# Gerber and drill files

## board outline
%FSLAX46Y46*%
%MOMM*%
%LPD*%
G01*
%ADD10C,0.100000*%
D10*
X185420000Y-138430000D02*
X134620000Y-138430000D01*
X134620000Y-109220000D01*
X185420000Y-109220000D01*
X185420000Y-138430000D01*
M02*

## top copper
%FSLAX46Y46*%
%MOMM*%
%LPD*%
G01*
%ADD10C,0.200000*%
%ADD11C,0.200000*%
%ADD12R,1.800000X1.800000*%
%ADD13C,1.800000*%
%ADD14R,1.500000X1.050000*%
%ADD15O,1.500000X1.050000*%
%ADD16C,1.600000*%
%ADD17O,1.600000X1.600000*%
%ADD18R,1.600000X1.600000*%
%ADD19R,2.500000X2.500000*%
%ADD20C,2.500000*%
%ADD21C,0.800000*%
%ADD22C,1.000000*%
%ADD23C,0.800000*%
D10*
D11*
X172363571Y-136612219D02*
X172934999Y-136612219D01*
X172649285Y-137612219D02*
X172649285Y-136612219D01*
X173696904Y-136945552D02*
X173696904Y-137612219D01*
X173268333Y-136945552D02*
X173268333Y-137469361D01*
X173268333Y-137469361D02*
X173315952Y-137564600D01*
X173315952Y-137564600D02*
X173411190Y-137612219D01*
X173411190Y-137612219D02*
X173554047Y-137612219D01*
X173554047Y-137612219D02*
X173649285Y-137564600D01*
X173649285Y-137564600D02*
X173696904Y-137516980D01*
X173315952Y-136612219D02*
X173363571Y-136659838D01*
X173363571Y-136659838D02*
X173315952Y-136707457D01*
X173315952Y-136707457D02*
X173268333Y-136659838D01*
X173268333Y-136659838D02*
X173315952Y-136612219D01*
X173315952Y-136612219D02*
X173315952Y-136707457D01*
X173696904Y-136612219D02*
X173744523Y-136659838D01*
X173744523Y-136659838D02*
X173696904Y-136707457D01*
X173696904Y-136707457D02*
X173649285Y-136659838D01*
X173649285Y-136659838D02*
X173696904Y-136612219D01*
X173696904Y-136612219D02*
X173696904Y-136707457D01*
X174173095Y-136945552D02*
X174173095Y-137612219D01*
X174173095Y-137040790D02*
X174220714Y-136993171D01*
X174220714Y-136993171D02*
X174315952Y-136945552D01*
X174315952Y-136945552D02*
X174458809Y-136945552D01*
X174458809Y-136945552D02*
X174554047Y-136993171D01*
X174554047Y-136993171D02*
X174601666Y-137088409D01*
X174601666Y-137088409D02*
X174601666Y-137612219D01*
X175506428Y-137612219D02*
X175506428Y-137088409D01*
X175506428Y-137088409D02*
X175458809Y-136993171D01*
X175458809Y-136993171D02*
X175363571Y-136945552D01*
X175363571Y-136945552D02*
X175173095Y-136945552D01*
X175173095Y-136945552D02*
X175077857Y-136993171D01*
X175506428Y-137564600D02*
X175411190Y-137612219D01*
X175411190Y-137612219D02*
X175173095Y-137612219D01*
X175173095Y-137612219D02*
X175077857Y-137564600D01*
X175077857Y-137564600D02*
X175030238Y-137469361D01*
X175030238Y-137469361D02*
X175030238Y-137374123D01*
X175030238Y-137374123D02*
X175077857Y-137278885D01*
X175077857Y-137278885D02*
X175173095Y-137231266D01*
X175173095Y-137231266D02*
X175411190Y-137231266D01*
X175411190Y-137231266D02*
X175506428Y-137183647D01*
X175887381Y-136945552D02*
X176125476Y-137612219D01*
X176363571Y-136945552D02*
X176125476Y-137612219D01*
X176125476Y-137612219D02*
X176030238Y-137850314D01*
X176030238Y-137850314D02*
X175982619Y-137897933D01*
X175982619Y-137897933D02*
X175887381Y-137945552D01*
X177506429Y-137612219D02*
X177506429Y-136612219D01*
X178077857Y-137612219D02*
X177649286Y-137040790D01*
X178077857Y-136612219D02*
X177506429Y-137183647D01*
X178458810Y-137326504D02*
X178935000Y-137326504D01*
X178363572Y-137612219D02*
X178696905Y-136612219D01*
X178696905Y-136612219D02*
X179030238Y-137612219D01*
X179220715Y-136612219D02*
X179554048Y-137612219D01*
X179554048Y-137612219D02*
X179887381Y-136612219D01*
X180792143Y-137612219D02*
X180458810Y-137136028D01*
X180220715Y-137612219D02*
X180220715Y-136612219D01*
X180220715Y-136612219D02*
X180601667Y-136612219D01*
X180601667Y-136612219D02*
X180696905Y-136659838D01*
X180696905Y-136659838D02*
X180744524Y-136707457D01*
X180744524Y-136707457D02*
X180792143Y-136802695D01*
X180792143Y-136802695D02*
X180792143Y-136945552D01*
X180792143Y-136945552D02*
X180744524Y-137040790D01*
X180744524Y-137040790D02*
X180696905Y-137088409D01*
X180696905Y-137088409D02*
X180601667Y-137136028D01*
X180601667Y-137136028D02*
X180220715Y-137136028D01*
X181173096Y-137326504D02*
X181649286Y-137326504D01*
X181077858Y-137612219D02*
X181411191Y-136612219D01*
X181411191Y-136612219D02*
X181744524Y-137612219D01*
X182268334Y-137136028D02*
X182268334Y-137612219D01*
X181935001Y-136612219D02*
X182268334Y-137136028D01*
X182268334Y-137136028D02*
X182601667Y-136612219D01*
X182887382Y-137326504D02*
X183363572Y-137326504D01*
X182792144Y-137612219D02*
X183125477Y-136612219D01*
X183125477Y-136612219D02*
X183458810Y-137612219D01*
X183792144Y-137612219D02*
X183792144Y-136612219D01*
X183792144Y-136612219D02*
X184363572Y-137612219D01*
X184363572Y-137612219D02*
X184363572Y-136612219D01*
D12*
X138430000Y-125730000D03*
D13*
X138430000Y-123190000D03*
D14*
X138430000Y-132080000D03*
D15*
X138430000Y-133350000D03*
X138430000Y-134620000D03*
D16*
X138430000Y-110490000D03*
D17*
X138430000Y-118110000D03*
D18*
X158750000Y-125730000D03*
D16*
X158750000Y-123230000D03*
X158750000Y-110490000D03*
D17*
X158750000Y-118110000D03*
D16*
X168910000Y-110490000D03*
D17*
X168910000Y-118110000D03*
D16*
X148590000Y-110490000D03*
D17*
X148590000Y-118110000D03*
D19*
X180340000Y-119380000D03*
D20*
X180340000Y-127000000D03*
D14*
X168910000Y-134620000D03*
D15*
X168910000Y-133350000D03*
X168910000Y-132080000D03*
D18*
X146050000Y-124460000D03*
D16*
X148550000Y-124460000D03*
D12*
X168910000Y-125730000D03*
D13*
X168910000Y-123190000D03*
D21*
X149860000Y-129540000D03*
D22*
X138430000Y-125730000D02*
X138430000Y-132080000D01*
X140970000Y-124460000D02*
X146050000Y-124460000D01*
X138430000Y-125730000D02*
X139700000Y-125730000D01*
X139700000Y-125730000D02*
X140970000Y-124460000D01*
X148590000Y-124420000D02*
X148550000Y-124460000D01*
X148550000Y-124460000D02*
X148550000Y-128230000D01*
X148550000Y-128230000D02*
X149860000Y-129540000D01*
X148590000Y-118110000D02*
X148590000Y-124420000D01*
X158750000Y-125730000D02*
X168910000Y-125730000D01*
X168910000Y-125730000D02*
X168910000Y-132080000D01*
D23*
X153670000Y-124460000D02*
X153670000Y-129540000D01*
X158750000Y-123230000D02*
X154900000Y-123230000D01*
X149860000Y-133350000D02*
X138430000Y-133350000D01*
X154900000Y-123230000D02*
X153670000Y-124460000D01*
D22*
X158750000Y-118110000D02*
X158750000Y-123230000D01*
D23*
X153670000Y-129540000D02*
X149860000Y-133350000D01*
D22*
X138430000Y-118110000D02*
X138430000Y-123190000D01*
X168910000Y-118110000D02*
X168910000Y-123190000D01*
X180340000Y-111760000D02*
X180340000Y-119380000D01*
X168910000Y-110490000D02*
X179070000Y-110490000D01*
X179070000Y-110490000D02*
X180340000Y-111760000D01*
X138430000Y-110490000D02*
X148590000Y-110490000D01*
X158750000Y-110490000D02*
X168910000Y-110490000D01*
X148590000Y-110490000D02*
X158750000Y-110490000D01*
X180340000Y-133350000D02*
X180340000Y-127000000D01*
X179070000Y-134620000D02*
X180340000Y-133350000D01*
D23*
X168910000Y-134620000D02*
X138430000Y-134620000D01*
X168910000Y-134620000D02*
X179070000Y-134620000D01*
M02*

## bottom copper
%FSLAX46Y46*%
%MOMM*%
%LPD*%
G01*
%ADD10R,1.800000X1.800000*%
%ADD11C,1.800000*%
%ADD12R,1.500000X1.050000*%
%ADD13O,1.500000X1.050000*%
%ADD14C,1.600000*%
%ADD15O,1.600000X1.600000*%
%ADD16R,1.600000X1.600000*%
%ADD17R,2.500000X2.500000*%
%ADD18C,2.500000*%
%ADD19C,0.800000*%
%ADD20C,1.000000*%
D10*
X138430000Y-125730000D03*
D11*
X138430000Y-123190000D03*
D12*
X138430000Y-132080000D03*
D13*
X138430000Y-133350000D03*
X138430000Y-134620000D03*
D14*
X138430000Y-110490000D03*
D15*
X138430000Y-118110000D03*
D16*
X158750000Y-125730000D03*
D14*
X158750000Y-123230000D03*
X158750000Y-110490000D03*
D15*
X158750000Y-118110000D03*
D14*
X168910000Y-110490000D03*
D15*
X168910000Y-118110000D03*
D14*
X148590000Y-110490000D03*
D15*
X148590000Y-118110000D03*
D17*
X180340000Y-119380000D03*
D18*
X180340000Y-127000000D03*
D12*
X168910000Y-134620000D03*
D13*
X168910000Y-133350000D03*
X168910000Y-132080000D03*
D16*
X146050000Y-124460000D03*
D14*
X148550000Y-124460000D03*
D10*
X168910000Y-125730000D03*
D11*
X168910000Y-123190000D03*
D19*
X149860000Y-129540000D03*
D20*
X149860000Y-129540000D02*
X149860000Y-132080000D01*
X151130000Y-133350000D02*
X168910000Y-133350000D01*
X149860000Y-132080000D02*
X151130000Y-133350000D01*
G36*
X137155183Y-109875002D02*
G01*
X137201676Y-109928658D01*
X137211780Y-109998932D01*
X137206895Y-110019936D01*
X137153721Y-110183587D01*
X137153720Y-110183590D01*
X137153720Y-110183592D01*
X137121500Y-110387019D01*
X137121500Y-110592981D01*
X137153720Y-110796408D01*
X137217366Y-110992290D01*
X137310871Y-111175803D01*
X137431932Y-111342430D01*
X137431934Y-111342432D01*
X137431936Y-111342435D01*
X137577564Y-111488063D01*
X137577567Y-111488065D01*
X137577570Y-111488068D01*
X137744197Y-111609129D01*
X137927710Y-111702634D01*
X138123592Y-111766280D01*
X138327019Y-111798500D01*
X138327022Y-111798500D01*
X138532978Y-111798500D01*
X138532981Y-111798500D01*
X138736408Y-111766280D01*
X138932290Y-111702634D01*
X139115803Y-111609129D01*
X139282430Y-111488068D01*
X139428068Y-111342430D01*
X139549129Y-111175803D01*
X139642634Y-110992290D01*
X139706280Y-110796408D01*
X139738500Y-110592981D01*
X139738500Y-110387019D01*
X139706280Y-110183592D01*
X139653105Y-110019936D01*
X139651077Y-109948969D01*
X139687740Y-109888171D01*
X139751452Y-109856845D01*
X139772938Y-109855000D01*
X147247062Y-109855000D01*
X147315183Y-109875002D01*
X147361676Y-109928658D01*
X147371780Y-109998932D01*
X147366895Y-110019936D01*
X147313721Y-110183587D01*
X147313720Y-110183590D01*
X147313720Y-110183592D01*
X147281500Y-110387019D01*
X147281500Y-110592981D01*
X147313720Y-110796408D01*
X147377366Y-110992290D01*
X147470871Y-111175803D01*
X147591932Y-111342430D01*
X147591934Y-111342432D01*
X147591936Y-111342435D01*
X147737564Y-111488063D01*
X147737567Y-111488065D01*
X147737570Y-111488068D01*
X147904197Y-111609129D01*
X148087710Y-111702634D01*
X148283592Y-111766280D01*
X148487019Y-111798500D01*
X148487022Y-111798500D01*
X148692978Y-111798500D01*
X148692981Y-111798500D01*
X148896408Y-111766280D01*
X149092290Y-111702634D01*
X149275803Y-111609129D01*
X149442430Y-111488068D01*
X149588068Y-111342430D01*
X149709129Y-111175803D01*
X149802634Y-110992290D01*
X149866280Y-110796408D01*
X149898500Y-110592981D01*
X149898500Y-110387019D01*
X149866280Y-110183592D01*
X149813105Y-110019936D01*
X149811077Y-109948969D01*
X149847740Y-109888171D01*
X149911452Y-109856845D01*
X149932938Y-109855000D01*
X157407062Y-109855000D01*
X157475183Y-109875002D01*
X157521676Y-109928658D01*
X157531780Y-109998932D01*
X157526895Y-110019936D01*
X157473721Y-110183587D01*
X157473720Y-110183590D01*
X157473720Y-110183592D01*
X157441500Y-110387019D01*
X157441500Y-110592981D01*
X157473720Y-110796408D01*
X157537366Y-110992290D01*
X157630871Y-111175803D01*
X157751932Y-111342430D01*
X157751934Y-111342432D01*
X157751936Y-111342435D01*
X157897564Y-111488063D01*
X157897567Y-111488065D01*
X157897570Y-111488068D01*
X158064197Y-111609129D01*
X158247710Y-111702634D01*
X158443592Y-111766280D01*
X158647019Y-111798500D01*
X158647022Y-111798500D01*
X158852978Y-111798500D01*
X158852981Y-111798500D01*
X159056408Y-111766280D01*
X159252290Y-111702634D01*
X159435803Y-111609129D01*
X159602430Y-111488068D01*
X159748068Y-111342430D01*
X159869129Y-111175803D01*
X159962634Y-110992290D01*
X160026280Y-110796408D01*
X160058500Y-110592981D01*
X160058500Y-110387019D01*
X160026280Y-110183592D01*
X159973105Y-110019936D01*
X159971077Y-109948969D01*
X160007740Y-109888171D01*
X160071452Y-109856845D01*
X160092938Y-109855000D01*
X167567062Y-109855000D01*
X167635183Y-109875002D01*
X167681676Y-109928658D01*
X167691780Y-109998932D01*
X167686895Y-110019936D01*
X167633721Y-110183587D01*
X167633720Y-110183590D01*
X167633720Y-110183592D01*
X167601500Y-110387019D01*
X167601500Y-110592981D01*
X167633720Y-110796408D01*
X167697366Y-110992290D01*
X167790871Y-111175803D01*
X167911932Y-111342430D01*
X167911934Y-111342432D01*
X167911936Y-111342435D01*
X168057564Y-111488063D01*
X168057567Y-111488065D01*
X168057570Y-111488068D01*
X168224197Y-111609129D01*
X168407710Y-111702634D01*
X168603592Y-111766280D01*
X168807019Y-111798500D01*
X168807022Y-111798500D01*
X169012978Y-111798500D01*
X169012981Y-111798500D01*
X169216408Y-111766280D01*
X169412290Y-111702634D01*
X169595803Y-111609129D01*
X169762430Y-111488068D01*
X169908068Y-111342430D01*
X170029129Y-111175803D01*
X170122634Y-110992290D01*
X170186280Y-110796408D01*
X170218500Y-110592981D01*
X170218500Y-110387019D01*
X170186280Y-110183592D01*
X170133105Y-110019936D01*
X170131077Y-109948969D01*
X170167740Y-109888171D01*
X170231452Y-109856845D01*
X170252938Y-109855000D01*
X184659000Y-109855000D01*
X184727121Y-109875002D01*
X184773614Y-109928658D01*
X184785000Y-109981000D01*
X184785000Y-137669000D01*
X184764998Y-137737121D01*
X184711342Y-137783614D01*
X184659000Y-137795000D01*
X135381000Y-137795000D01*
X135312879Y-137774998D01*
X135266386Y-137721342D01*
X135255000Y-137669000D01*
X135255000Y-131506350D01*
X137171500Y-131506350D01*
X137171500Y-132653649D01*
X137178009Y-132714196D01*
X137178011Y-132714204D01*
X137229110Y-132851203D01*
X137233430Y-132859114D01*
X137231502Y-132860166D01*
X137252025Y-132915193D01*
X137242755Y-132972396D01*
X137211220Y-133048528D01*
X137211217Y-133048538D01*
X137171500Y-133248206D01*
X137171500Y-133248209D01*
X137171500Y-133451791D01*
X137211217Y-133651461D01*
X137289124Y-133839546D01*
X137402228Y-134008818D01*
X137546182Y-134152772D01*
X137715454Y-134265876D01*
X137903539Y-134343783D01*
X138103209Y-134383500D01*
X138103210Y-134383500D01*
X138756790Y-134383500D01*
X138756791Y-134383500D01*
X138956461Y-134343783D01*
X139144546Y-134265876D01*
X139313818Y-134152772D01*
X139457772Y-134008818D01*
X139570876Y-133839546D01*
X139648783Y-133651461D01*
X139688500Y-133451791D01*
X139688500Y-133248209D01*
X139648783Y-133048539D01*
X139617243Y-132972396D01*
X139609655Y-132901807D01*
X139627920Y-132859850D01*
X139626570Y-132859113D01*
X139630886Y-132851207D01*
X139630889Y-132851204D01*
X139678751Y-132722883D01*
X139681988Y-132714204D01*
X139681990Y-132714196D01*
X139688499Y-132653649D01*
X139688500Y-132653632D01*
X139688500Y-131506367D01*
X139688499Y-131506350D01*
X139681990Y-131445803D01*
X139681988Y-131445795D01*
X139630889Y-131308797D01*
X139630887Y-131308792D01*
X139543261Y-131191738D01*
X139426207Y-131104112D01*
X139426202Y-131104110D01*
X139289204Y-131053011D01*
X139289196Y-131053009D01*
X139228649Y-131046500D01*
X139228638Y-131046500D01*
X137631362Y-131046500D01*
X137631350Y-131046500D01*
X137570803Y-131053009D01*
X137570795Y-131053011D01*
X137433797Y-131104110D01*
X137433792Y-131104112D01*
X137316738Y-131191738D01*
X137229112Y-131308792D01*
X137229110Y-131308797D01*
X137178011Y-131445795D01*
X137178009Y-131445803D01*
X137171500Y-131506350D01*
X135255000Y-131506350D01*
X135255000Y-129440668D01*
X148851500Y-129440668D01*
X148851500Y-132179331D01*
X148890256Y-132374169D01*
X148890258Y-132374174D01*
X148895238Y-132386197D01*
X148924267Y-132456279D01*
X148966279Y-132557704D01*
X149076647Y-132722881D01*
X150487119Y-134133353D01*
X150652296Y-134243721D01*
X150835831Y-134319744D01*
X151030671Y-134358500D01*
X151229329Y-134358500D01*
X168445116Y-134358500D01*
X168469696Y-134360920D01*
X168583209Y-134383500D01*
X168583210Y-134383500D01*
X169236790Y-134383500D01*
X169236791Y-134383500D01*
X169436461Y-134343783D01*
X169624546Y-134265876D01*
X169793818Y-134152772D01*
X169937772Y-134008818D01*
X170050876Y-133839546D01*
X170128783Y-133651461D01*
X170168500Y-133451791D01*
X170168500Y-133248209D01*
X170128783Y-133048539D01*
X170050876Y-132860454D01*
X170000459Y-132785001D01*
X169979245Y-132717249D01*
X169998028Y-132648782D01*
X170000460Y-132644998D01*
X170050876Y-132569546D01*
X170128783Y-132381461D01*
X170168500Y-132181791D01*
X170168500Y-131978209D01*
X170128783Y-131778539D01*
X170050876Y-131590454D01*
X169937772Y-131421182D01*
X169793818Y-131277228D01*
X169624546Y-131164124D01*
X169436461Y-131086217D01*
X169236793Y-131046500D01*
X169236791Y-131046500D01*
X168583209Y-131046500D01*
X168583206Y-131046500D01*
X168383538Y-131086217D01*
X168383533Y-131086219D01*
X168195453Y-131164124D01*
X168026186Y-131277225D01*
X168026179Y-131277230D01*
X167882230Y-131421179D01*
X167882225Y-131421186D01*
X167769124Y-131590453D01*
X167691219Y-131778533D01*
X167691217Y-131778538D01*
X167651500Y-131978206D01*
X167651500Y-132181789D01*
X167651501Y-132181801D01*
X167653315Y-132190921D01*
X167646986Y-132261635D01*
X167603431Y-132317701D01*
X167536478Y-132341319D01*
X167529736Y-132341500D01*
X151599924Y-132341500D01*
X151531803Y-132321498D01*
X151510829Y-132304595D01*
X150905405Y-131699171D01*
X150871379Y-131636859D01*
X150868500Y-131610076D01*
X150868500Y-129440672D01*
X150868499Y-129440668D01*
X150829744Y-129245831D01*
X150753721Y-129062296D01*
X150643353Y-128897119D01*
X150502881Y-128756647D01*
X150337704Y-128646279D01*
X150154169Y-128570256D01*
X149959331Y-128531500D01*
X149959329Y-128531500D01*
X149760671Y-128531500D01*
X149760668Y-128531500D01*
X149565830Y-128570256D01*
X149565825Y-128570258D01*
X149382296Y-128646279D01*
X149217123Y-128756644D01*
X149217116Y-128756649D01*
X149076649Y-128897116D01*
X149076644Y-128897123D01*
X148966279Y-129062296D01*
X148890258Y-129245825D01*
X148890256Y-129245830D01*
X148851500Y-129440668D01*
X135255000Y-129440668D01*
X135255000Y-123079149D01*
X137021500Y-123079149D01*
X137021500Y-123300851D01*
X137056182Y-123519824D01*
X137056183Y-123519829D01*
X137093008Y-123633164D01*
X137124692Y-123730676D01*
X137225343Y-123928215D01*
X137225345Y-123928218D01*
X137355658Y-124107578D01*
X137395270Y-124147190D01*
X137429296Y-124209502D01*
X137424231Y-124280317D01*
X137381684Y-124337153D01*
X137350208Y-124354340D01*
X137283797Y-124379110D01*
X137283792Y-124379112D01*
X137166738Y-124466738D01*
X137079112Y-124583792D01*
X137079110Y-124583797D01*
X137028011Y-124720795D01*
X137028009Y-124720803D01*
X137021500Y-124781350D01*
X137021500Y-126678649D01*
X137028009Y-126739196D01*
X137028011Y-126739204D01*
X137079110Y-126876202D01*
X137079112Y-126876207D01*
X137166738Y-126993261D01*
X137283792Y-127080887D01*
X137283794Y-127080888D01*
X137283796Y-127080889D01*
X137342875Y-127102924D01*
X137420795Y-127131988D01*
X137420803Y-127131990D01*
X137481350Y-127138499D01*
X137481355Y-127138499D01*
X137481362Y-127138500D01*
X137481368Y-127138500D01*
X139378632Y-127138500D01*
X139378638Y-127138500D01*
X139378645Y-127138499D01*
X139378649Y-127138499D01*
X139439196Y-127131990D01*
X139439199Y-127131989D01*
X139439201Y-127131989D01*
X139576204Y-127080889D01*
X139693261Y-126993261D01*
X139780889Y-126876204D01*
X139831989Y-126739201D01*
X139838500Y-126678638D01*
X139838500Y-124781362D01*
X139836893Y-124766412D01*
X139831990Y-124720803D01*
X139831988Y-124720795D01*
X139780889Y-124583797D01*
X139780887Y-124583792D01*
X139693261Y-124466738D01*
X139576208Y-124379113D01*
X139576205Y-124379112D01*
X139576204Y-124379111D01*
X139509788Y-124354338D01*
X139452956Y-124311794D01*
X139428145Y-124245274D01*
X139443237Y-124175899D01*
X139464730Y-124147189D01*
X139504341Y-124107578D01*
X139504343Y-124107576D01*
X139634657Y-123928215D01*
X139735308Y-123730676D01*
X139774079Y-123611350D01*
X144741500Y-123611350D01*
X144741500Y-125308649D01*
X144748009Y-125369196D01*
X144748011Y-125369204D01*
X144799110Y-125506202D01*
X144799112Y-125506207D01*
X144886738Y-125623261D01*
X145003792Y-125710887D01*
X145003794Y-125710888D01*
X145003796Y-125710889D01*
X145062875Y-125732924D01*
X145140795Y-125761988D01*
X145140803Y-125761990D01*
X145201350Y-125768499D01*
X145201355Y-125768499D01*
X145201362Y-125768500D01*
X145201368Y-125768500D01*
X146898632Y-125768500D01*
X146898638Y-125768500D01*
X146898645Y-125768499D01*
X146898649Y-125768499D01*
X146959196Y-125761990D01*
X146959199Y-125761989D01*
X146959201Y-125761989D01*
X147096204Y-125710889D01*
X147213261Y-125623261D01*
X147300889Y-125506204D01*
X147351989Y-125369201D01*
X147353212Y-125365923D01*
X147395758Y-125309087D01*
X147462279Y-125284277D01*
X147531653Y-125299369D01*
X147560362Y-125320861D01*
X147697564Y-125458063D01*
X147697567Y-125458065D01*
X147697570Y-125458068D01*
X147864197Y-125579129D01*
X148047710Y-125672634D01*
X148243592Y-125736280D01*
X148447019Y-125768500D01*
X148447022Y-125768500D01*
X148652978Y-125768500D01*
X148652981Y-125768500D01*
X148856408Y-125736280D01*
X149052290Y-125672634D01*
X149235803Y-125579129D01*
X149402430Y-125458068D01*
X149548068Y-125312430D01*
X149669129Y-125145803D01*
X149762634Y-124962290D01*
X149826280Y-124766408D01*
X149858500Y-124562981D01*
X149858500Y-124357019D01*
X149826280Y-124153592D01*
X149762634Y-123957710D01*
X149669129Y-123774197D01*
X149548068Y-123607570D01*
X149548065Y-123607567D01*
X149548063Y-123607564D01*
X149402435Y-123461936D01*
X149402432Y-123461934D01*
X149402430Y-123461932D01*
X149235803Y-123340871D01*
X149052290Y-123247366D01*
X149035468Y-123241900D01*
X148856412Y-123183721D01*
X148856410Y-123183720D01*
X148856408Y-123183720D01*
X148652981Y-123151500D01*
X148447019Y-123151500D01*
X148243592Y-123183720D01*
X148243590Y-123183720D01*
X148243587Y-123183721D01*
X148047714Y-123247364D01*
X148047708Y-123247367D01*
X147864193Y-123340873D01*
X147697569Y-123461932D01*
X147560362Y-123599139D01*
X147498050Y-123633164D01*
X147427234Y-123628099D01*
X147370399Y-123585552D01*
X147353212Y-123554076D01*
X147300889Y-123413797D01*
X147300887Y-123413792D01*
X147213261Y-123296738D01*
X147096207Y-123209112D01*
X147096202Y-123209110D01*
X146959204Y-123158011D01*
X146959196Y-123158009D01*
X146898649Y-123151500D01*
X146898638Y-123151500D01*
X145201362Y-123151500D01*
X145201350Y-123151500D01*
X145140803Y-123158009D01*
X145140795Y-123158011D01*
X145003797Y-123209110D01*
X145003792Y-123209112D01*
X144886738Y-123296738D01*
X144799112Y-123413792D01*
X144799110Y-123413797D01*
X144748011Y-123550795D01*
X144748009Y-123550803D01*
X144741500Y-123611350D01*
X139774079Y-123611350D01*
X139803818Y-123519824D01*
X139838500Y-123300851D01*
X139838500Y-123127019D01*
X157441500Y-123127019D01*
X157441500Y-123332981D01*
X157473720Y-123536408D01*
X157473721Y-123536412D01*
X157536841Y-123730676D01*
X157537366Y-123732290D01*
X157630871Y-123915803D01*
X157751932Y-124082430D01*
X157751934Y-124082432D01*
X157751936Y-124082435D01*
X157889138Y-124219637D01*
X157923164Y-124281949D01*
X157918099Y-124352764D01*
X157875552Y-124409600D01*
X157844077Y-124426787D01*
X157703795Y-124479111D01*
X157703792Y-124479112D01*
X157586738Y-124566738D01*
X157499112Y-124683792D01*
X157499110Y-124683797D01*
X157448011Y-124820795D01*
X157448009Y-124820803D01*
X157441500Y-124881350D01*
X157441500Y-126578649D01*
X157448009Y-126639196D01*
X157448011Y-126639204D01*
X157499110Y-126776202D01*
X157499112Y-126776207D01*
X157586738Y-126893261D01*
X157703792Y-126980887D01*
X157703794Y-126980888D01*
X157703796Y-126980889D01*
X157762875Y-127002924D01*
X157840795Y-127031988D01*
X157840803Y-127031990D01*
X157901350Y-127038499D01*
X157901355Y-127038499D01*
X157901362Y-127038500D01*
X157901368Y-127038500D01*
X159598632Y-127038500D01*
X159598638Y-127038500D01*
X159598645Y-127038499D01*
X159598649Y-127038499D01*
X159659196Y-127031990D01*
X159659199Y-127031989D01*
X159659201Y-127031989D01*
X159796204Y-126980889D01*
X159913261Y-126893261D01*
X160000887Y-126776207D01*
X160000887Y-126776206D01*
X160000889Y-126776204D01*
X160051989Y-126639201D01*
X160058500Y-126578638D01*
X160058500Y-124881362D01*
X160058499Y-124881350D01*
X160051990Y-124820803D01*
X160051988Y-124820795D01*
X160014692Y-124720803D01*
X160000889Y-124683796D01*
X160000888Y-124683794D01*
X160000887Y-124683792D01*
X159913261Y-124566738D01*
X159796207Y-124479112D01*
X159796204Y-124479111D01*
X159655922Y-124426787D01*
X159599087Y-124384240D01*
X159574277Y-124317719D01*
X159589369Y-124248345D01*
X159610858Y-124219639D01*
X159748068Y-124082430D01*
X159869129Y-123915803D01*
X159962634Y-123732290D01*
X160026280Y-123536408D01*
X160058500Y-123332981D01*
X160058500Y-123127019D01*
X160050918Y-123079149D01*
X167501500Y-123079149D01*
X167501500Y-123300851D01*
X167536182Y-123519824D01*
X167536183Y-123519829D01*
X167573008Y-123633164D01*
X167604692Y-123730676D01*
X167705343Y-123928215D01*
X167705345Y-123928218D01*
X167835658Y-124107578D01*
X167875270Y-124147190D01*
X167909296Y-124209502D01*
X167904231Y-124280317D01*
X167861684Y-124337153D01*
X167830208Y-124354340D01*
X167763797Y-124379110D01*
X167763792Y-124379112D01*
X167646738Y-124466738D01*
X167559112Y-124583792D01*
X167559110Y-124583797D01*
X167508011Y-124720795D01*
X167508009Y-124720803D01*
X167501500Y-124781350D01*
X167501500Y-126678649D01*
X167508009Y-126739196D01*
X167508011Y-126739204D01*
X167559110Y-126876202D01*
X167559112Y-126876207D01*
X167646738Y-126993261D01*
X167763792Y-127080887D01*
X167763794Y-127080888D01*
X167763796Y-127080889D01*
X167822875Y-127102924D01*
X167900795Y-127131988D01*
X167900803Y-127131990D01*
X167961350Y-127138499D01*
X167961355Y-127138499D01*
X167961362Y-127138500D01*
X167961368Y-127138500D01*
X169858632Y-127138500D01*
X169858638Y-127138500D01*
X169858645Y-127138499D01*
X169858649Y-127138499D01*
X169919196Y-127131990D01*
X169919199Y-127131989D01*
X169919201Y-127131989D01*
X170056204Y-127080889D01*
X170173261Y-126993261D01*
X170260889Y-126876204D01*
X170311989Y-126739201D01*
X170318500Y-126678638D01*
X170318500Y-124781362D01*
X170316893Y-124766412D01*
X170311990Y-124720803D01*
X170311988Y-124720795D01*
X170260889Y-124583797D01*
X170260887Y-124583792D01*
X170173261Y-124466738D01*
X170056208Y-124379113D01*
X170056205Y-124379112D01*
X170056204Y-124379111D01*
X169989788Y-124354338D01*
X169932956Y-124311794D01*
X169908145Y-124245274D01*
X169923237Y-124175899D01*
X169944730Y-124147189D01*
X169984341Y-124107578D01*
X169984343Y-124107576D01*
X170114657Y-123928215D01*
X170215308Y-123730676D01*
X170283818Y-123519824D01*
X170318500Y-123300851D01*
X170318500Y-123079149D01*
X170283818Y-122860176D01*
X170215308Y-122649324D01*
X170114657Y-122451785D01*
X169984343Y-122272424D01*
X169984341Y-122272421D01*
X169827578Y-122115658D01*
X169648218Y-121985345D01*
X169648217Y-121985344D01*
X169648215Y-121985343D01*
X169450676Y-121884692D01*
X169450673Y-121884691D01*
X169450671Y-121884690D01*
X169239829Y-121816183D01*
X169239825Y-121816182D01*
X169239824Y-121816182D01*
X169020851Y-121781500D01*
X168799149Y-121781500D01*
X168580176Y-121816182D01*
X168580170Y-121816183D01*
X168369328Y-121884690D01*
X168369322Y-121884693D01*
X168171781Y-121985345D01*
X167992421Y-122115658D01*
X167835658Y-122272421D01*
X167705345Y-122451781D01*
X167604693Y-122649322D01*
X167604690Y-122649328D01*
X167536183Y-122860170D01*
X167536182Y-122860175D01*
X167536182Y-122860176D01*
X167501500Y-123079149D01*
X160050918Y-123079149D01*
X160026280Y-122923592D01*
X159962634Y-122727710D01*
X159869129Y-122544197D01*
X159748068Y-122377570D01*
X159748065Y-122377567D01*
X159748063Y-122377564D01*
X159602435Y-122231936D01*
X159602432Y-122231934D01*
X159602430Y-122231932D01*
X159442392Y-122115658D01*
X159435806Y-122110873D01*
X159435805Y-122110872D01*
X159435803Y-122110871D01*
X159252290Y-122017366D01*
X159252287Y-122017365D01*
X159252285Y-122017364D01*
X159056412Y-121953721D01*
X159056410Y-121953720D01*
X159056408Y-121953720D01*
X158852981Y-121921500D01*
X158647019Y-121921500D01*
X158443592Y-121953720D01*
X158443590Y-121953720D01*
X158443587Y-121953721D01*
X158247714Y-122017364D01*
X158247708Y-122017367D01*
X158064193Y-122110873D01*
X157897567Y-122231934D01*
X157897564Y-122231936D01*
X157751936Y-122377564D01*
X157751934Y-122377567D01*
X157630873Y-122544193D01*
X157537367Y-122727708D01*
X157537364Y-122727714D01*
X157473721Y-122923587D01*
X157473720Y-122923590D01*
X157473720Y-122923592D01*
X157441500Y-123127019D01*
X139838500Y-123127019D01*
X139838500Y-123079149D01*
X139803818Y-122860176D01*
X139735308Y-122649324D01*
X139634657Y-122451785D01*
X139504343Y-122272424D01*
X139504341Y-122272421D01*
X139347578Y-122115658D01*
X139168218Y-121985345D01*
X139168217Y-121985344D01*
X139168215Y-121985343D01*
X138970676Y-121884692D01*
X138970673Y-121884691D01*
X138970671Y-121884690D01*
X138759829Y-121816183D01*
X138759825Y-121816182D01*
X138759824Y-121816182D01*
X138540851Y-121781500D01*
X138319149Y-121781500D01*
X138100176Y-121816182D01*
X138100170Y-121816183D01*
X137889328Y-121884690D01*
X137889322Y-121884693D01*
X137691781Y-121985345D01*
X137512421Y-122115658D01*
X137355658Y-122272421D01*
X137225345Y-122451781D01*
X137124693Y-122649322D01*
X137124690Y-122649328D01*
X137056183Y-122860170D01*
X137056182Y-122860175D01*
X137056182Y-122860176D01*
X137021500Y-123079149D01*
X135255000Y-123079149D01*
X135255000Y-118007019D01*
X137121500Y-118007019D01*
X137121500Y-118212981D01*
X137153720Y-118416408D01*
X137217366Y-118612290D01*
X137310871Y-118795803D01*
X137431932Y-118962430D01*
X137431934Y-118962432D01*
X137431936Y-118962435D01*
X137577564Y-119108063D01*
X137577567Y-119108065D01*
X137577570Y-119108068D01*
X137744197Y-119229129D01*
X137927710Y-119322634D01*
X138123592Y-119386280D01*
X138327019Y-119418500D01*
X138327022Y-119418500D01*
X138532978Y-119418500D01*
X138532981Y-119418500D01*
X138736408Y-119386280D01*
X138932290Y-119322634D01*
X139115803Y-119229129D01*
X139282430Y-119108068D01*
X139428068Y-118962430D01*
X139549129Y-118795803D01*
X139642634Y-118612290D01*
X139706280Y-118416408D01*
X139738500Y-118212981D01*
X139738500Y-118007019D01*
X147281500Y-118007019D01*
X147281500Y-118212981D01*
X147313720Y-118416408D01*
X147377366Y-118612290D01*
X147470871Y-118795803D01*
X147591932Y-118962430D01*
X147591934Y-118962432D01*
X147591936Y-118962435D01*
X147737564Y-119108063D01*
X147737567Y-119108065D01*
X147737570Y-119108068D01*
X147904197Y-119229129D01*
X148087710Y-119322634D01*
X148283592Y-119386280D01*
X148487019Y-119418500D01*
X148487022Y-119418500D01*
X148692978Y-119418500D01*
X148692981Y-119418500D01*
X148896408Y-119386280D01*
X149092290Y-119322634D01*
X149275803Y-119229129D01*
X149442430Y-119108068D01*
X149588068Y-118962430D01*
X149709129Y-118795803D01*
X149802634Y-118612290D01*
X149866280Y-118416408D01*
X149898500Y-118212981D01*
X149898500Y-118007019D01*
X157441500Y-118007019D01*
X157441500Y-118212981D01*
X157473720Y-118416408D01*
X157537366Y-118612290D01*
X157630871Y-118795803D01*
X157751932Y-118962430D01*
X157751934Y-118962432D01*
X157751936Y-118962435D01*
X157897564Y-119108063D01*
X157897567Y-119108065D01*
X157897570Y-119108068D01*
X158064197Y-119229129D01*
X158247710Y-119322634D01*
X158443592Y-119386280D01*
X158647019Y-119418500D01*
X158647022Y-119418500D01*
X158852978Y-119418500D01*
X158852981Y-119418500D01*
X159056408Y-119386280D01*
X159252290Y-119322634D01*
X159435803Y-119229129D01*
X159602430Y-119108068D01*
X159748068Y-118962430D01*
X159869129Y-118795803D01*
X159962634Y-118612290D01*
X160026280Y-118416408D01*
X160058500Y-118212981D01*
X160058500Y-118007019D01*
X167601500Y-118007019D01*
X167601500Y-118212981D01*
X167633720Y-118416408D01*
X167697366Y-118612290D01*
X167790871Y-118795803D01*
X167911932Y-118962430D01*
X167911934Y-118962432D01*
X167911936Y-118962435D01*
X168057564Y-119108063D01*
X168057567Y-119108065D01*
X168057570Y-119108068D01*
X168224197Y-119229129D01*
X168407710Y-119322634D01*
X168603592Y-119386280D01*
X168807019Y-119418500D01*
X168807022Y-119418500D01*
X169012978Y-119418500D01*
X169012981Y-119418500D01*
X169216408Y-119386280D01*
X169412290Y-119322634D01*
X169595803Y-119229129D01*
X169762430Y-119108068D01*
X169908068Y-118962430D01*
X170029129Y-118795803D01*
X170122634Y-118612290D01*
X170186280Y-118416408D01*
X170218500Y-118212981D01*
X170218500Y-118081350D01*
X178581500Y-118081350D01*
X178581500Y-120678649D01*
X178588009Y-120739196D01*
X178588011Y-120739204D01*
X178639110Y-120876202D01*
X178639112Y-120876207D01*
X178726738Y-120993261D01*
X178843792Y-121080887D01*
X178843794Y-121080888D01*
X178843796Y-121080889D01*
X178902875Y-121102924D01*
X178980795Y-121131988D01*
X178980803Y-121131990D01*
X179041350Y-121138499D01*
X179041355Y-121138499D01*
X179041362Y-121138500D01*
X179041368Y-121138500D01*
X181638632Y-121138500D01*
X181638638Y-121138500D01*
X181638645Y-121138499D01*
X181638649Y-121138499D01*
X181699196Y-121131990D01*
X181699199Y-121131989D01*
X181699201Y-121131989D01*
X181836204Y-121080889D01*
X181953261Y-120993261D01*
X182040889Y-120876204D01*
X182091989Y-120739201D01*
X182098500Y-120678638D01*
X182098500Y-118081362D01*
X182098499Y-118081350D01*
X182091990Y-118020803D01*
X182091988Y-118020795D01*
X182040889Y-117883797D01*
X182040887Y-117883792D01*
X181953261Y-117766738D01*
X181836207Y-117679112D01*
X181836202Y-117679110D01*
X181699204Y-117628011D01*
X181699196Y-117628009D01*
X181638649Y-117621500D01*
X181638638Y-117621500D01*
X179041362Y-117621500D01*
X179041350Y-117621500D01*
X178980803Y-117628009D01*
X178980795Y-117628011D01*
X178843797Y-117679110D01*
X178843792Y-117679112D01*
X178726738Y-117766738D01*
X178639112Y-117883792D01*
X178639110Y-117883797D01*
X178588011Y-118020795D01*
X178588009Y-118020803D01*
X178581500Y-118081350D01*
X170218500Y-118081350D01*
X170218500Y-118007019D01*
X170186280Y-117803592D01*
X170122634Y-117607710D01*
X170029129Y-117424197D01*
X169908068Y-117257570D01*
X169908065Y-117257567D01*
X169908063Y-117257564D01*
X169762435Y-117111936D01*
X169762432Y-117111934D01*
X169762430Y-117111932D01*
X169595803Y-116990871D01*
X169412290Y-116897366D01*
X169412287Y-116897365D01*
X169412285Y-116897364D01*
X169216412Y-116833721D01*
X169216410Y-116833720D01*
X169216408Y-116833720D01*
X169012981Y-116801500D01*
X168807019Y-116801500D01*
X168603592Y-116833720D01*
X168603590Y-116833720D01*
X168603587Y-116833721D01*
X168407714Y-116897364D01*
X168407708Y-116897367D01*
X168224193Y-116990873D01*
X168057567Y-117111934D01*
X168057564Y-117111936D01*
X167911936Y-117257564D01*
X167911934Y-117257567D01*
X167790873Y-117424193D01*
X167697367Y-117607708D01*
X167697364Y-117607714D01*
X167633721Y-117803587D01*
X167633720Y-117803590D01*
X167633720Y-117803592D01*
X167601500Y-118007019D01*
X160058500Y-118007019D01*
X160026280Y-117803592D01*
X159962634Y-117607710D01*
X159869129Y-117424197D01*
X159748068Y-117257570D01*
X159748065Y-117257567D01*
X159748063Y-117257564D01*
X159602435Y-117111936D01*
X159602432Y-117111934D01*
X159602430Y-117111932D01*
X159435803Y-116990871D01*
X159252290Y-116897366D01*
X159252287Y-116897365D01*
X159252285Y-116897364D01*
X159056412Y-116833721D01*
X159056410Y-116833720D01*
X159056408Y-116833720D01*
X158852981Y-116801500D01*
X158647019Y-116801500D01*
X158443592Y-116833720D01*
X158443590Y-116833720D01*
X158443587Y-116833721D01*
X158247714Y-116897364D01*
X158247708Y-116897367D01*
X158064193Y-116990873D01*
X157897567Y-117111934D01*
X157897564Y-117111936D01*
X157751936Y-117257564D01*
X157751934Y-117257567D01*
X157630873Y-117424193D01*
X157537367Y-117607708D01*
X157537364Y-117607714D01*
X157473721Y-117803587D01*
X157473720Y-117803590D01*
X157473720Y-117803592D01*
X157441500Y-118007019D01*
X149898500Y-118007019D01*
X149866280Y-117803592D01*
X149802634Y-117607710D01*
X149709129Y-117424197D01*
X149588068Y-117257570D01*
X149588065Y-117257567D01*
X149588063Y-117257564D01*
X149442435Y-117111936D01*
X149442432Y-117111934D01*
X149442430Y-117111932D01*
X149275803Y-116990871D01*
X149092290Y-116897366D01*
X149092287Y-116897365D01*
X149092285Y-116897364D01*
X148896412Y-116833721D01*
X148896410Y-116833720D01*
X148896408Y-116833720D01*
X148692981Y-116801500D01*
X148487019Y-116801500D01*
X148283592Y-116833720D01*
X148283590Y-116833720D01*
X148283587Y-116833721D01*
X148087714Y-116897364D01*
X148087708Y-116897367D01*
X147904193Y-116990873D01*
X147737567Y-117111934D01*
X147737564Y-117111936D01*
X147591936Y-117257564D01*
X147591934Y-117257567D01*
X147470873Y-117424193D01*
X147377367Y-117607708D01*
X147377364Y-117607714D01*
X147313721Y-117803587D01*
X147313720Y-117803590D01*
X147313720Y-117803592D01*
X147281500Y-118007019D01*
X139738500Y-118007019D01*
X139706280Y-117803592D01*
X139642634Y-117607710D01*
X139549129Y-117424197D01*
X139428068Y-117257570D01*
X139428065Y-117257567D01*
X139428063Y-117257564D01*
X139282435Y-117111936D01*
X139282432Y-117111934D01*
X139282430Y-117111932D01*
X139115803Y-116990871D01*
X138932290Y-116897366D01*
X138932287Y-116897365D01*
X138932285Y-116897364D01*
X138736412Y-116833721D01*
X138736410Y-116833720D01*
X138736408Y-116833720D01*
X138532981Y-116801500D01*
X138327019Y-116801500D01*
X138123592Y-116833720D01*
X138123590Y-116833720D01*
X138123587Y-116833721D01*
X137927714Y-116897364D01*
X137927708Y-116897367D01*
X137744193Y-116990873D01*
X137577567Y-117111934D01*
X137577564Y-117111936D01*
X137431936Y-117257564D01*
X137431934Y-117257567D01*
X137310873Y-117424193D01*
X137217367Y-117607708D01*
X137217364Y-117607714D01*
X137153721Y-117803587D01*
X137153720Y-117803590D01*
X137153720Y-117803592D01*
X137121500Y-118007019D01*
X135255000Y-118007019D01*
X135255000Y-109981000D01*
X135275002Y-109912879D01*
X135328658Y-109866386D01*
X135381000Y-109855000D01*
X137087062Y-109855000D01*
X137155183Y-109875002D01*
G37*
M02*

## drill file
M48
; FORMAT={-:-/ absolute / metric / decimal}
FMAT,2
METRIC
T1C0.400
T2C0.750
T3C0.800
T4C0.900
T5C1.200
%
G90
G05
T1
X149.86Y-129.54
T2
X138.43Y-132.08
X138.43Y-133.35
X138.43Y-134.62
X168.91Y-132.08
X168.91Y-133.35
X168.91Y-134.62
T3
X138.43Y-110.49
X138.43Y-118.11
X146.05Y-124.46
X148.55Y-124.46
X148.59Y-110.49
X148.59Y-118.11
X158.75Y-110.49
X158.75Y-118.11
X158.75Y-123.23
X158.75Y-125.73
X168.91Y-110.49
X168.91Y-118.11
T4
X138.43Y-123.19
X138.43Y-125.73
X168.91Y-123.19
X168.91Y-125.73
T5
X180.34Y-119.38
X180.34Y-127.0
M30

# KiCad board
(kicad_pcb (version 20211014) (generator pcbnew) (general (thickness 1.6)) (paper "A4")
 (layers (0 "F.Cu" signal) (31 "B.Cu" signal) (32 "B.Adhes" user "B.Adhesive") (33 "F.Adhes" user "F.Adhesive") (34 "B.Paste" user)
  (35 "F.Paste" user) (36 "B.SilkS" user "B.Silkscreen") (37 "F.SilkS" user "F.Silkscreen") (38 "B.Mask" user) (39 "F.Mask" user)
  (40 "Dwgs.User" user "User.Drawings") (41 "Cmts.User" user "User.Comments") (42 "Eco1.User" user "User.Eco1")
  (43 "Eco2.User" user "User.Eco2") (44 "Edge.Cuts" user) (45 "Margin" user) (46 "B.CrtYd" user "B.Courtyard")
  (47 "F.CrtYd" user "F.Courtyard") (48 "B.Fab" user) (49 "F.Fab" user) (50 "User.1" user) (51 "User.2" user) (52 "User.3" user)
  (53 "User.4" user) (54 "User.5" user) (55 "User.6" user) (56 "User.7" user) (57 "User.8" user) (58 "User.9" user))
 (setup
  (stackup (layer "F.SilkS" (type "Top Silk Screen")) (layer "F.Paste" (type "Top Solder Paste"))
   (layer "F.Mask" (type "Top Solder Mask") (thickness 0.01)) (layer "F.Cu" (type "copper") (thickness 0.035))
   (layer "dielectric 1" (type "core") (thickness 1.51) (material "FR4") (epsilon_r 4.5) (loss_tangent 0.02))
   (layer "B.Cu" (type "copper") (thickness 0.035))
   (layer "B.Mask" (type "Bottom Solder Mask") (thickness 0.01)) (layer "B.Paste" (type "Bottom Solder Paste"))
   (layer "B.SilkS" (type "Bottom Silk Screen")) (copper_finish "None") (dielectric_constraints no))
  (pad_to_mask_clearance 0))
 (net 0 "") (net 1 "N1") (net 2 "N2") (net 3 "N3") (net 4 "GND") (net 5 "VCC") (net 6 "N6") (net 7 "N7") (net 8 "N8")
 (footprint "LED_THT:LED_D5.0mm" (layer "F.Cu") (at 138.43 125.73 90)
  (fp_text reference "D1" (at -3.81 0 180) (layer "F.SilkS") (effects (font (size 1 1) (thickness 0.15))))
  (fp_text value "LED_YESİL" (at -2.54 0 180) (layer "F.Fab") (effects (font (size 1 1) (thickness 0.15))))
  (pad "1" thru_hole rect (at 0 0 90) (size 1.8 1.8) (drill 0.9) (layers *.Cu *.Mask) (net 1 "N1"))
  (pad "2" thru_hole circle (at 2.54 0 90) (size 1.8 1.8) (drill 0.9) (layers *.Cu *.Mask) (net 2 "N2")))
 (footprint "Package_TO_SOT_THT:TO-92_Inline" (layer "F.Cu") (at 138.43 132.08 -90)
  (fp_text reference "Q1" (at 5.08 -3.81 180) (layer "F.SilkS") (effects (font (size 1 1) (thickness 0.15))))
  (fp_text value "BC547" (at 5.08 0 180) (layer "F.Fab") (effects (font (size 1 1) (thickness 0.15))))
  (pad "1" thru_hole rect (at 0 0 270) (size 1.05 1.5) (drill 0.75) (layers *.Cu *.Mask) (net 1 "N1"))
  (pad "2" thru_hole oval (at 1.27 0 270) (size 1.05 1.5) (drill 0.75) (layers *.Cu *.Mask) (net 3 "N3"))
  (pad "3" thru_hole oval (at 2.54 0 270) (size 1.05 1.5) (drill 0.75) (layers *.Cu *.Mask) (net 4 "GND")))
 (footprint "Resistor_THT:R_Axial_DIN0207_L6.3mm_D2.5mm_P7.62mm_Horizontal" (layer "F.Cu") (at 138.43 110.49 -90)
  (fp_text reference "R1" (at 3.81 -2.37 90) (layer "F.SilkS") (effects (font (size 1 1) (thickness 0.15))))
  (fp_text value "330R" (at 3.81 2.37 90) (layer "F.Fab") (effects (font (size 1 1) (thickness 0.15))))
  (pad "1" thru_hole circle (at 0 0 270) (size 1.6 1.6) (drill 0.8) (layers *.Cu *.Mask) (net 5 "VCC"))
  (pad "2" thru_hole oval (at 7.62 0 270) (size 1.6 1.6) (drill 0.8) (layers *.Cu *.Mask) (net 2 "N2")))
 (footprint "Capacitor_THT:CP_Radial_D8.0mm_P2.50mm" (layer "F.Cu") (at 158.75 125.73 90)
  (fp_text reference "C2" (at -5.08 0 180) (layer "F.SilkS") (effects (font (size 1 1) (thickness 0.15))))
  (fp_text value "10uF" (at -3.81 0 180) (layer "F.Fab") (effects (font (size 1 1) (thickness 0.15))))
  (pad "1" thru_hole rect (at 0 0 90) (size 1.6 1.6) (drill 0.8) (layers *.Cu *.Mask) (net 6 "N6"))
  (pad "2" thru_hole circle (at 2.5 0 90) (size 1.6 1.6) (drill 0.8) (layers *.Cu *.Mask) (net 3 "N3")))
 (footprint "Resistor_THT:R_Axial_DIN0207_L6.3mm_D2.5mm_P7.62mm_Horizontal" (layer "F.Cu") (at 158.75 110.49 -90)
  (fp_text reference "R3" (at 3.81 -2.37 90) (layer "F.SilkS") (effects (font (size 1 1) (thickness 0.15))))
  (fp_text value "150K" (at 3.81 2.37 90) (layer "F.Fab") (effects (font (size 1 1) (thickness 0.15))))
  (pad "1" thru_hole circle (at 0 0 270) (size 1.6 1.6) (drill 0.8) (layers *.Cu *.Mask) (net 5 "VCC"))
  (pad "2" thru_hole oval (at 7.62 0 270) (size 1.6 1.6) (drill 0.8) (layers *.Cu *.Mask) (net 3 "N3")))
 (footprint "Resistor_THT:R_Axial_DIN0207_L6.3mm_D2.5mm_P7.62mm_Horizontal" (layer "F.Cu") (at 168.91 110.49 -90)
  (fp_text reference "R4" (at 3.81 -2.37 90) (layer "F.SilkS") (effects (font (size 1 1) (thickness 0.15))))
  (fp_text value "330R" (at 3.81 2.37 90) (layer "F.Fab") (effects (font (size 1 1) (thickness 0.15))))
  (pad "1" thru_hole circle (at 0 0 270) (size 1.6 1.6) (drill 0.8) (layers *.Cu *.Mask) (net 5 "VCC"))
  (pad "2" thru_hole oval (at 7.62 0 270) (size 1.6 1.6) (drill 0.8) (layers *.Cu *.Mask) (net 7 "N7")))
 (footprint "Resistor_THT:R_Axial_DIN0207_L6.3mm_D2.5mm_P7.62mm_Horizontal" (layer "F.Cu") (at 148.59 110.49 -90)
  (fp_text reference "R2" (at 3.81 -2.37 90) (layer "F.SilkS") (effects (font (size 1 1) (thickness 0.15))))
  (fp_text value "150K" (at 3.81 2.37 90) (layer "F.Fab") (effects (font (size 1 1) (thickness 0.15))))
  (pad "1" thru_hole circle (at 0 0 270) (size 1.6 1.6) (drill 0.8) (layers *.Cu *.Mask) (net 5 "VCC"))
  (pad "2" thru_hole oval (at 7.62 0 270) (size 1.6 1.6) (drill 0.8) (layers *.Cu *.Mask) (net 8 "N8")))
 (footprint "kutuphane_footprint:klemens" (layer "F.Cu") (at 180.34 121.92 -90)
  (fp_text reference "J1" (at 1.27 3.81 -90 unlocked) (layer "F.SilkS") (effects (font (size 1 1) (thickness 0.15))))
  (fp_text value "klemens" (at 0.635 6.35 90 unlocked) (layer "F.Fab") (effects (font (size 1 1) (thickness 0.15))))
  (pad "1" thru_hole rect (at -2.54 0 270) (size 2.5 2.5) (drill 1.2) (layers *.Cu *.Mask) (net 5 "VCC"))
  (pad "2" thru_hole circle (at 5.08 0 270) (size 2.5 2.5) (drill 1.2) (layers *.Cu *.Mask) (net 4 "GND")))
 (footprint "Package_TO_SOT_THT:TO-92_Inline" (layer "F.Cu") (at 168.91 134.62 90)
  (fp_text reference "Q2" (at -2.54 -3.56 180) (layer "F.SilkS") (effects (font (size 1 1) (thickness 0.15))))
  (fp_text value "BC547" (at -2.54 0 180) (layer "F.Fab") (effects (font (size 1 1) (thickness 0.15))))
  (pad "1" thru_hole rect (at 0 0 90) (size 1.05 1.5) (drill 0.75) (layers *.Cu *.Mask) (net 4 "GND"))
  (pad "2" thru_hole oval (at 1.27 0 90) (size 1.05 1.5) (drill 0.75) (layers *.Cu *.Mask) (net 8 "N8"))
  (pad "3" thru_hole oval (at 2.54 0 90) (size 1.05 1.5) (drill 0.75) (layers *.Cu *.Mask) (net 6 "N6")))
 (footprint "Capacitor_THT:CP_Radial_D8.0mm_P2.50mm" (layer "F.Cu") (at 146.05 124.46)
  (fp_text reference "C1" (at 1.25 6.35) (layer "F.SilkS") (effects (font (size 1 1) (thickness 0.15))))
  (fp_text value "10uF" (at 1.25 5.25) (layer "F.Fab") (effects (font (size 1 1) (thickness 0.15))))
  (pad "1" thru_hole rect (at 0 0) (size 1.6 1.6) (drill 0.8) (layers *.Cu *.Mask) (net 1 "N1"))
  (pad "2" thru_hole circle (at 2.5 0) (size 1.6 1.6) (drill 0.8) (layers *.Cu *.Mask) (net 8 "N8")))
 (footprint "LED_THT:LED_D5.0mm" (layer "F.Cu") (at 168.91 125.73 90)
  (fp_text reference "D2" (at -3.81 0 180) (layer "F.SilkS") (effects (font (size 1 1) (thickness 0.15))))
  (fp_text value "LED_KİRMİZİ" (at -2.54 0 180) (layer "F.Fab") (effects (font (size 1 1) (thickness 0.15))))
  (pad "1" thru_hole rect (at 0 0 90) (size 1.8 1.8) (drill 0.9) (layers *.Cu *.Mask) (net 6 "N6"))
  (pad "2" thru_hole circle (at 2.54 0 90) (size 1.8 1.8) (drill 0.9) (layers *.Cu *.Mask) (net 7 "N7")))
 (gr_poly (pts (xy 185.42 138.43) (xy 134.62 138.43) (xy 134.62 109.22) (xy 185.42 109.22)) (layer "Edge.Cuts") (width 0.1) (fill none))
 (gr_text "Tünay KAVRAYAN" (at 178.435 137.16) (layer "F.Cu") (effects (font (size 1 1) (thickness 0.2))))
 (segment (start 138.43 125.73) (end 138.43 132.08) (width 1) (layer "F.Cu") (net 1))
 (segment (start 140.97 124.46) (end 146.05 124.46) (width 1) (layer "F.Cu") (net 1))
 (segment (start 138.43 125.73) (end 139.7 125.73) (width 1) (layer "F.Cu") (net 1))
 (segment (start 139.7 125.73) (end 140.97 124.46) (width 1) (layer "F.Cu") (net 1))
 (segment (start 148.59 124.42) (end 148.55 124.46) (width 1) (layer "F.Cu") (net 8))
 (segment (start 148.55 124.46) (end 148.55 128.23) (width 1) (layer "F.Cu") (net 8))
 (segment (start 148.55 128.23) (end 149.86 129.54) (width 1) (layer "F.Cu") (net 8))
 (segment (start 148.59 118.11) (end 148.59 124.42) (width 1) (layer "F.Cu") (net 8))
 (via (at 149.86 129.54) (size 0.8) (drill 0.4) (layers "F.Cu" "B.Cu") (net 8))
 (segment (start 149.86 129.54) (end 149.86 132.08) (width 1) (layer "B.Cu") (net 8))
 (segment (start 151.13 133.35) (end 168.91 133.35) (width 1) (layer "B.Cu") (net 8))
 (segment (start 149.86 132.08) (end 151.13 133.35) (width 1) (layer "B.Cu") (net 8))
 (segment (start 158.75 125.73) (end 168.91 125.73) (width 1) (layer "F.Cu") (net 6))
 (segment (start 168.91 125.73) (end 168.91 132.08) (width 1) (layer "F.Cu") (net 6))
 (segment (start 153.67 124.46) (end 153.67 129.54) (width 0.8) (layer "F.Cu") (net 3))
 (segment (start 158.75 123.23) (end 154.9 123.23) (width 0.8) (layer "F.Cu") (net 3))
 (segment (start 149.86 133.35) (end 138.43 133.35) (width 0.8) (layer "F.Cu") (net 3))
 (segment (start 154.9 123.23) (end 153.67 124.46) (width 0.8) (layer "F.Cu") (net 3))
 (segment (start 158.75 118.11) (end 158.75 123.23) (width 1) (layer "F.Cu") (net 3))
 (segment (start 153.67 129.54) (end 149.86 133.35) (width 0.8) (layer "F.Cu") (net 3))
 (segment (start 138.43 118.11) (end 138.43 123.19) (width 1) (layer "F.Cu") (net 2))
 (segment (start 168.91 118.11) (end 168.91 123.19) (width 1) (layer "F.Cu") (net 7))
 (segment (start 180.34 111.76) (end 180.34 119.38) (width 1) (layer "F.Cu") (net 5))
 (segment (start 168.91 110.49) (end 179.07 110.49) (width 1) (layer "F.Cu") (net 5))
 (segment (start 179.07 110.49) (end 180.34 111.76) (width 1) (layer "F.Cu") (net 5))
 (segment (start 138.43 110.49) (end 148.59 110.49) (width 1) (layer "F.Cu") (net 5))
 (segment (start 158.75 110.49) (end 168.91 110.49) (width 1) (layer "F.Cu") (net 5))
 (segment (start 148.59 110.49) (end 158.75 110.49) (width 1) (layer "F.Cu") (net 5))
 (segment (start 180.34 133.35) (end 180.34 127) (width 1) (layer "F.Cu") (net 4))
 (segment (start 179.07 134.62) (end 180.34 133.35) (width 1) (layer "F.Cu") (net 4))
 (segment (start 168.91 134.62) (end 138.43 134.62) (width 0.8) (layer "F.Cu") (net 4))
 (segment (start 168.91 134.62) (end 179.07 134.62) (width 0.8) (layer "F.Cu") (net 4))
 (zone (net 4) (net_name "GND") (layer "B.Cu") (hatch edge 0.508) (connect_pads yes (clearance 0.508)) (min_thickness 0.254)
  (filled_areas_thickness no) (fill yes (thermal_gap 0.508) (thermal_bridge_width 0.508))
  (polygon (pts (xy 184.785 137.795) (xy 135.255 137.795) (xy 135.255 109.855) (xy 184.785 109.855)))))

